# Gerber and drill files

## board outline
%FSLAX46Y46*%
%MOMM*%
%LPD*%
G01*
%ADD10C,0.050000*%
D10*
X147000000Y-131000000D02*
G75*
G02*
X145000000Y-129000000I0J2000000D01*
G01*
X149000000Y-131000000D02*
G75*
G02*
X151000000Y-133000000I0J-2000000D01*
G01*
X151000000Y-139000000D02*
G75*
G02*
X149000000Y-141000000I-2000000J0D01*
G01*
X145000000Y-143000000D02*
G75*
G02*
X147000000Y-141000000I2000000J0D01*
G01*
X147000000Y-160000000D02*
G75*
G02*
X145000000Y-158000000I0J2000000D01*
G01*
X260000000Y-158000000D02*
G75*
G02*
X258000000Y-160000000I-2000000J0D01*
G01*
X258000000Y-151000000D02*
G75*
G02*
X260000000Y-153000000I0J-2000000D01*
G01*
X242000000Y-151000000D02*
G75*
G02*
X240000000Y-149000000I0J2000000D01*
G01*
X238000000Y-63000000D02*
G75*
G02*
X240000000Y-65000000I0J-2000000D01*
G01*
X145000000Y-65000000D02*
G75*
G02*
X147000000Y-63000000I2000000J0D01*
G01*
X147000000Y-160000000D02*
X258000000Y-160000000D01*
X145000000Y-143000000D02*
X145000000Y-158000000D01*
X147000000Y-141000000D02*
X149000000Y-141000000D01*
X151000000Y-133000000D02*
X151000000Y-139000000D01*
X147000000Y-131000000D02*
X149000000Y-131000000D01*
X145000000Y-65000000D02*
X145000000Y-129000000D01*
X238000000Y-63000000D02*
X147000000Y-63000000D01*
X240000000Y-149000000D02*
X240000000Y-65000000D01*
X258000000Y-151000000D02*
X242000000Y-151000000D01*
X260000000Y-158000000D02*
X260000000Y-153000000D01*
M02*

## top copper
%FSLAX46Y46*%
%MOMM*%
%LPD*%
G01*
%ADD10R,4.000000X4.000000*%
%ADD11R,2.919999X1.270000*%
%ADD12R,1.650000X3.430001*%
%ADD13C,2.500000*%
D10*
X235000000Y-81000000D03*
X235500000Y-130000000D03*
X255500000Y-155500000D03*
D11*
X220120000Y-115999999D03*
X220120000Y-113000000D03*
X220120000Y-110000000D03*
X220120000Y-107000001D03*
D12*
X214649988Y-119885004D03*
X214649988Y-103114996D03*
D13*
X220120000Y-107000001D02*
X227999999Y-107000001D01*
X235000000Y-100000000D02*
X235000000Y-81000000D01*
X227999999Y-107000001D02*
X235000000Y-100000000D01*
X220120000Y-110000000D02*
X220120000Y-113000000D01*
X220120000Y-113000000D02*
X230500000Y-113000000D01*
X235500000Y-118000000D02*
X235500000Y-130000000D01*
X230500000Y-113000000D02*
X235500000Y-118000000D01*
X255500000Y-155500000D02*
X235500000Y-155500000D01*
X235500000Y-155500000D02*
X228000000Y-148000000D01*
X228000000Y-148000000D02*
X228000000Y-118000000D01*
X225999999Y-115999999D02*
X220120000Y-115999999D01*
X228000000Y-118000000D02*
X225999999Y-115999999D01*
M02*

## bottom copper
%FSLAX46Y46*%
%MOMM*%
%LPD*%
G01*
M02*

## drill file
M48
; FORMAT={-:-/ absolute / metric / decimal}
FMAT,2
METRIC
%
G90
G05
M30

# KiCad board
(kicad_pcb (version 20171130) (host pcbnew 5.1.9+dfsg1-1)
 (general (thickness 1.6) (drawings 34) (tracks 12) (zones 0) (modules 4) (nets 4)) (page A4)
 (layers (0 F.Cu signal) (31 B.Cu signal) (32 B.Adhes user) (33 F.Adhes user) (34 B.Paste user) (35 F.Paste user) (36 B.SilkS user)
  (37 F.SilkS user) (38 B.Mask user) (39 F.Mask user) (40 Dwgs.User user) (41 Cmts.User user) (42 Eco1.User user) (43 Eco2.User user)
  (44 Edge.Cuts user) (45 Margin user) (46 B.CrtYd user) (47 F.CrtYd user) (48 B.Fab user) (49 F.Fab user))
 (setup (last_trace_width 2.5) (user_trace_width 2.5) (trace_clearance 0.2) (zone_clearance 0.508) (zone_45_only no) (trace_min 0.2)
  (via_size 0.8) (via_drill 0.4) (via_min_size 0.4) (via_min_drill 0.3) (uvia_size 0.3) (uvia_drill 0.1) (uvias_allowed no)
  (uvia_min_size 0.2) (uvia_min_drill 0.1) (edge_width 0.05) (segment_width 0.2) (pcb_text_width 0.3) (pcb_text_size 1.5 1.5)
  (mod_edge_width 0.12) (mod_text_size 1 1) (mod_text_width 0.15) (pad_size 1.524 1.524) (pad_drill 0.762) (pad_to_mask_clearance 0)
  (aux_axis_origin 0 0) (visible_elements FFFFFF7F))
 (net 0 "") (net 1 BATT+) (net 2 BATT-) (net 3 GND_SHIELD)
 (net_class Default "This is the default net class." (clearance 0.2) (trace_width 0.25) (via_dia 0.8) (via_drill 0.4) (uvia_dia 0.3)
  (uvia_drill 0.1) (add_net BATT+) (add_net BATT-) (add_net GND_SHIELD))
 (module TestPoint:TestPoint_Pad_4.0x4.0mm (layer F.Cu) (at 235 81)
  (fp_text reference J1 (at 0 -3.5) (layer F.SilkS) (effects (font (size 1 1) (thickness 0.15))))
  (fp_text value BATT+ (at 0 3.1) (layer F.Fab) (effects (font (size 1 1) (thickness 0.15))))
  (pad 1 smd rect (at 0 0) (size 4 4) (layers F.Cu F.Mask) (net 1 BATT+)))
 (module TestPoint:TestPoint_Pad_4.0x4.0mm (layer F.Cu) (at 235.5 130)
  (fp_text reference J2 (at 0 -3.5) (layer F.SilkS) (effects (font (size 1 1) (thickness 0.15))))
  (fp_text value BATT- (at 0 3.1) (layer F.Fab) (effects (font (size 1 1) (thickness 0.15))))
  (pad 1 smd rect (at 0 0) (size 4 4) (layers F.Cu F.Mask) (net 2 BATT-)))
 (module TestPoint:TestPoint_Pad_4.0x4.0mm (layer F.Cu) (at 255.5 155.5)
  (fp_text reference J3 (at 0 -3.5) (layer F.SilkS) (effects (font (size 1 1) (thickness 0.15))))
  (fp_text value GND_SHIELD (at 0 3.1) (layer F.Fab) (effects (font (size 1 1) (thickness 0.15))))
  (pad 1 smd rect (at 0 0) (size 4 4) (layers F.Cu F.Mask) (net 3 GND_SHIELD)))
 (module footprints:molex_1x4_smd (layer F.Cu) (at 215 111.5 270)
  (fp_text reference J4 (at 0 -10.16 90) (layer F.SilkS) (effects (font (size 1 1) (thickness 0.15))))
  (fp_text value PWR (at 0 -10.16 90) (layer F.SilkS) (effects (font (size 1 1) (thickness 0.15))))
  (pad 1 smd rect (at 4.499999 -5.12 270) (size 1.27 2.919999) (layers F.Cu F.Paste F.Mask) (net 3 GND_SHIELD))
  (pad 2 smd rect (at 1.5 -5.12 270) (size 1.27 2.919999) (layers F.Cu F.Paste F.Mask) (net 2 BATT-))
  (pad 3 smd rect (at -1.5 -5.12 270) (size 1.27 2.919999) (layers F.Cu F.Paste F.Mask) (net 2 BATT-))
  (pad 4 smd rect (at -4.499999 -5.12 270) (size 1.27 2.919999) (layers F.Cu F.Paste F.Mask) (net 1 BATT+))
  (pad P1 smd rect (at 8.385004 0.350012 270) (size 3.430001 1.65) (layers F.Cu F.Paste F.Mask))
  (pad P2 smd rect (at -8.385004 0.350012 270) (size 3.430001 1.65) (layers F.Cu F.Paste F.Mask)))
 (gr_arc (start 147 129) (end 145 129) (angle -90) (layer Edge.Cuts) (width 0.05))
 (gr_arc (start 149 133) (end 151 133) (angle -90) (layer Edge.Cuts) (width 0.05))
 (gr_arc (start 149 139) (end 149 141) (angle -90) (layer Edge.Cuts) (width 0.05))
 (gr_arc (start 147 143) (end 147 141) (angle -90) (layer Edge.Cuts) (width 0.05))
 (gr_arc (start 147 158) (end 145 158) (angle -90) (layer Edge.Cuts) (width 0.05))
 (gr_arc (start 258 158) (end 258 160) (angle -90) (layer Edge.Cuts) (width 0.05))
 (gr_arc (start 258 153) (end 260 153) (angle -90) (layer Edge.Cuts) (width 0.05))
 (gr_arc (start 242 149) (end 240 149) (angle -90) (layer Edge.Cuts) (width 0.05))
 (gr_arc (start 238 65) (end 240 65) (angle -90) (layer Edge.Cuts) (width 0.05))
 (gr_arc (start 147 65) (end 147 63) (angle -90) (layer Edge.Cuts) (width 0.05))
 (gr_line (start 147 160) (end 258 160) (layer Edge.Cuts) (width 0.05))
 (gr_line (start 145 143) (end 145 158) (layer Edge.Cuts) (width 0.05))
 (gr_line (start 147 141) (end 149 141) (layer Edge.Cuts) (width 0.05))
 (gr_line (start 151 133) (end 151 139) (layer Edge.Cuts) (width 0.05))
 (gr_line (start 147 131) (end 149 131) (layer Edge.Cuts) (width 0.05))
 (gr_line (start 145 65) (end 145 129) (layer Edge.Cuts) (width 0.05))
 (gr_line (start 238 63) (end 147 63) (layer Edge.Cuts) (width 0.05))
 (gr_line (start 240 149) (end 240 65) (layer Edge.Cuts) (width 0.05))
 (gr_line (start 258 151) (end 242 151) (layer Edge.Cuts) (width 0.05))
 (gr_line (start 260 158) (end 260 153) (layer Edge.Cuts) (width 0.05))
 (segment (start 220.12 107.000001) (end 227.999999 107.000001) (width 2.5) (layer F.Cu) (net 1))
 (segment (start 235 100) (end 235 81) (width 2.5) (layer F.Cu) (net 1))
 (segment (start 227.999999 107.000001) (end 235 100) (width 2.5) (layer F.Cu) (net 1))
 (segment (start 220.12 110) (end 220.12 113) (width 2.5) (layer F.Cu) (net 2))
 (segment (start 220.12 113) (end 230.5 113) (width 2.5) (layer F.Cu) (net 2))
 (segment (start 235.5 118) (end 235.5 130) (width 2.5) (layer F.Cu) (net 2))
 (segment (start 230.5 113) (end 235.5 118) (width 2.5) (layer F.Cu) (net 2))
 (segment (start 255.5 155.5) (end 235.5 155.5) (width 2.5) (layer F.Cu) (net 3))
 (segment (start 235.5 155.5) (end 228 148) (width 2.5) (layer F.Cu) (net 3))
 (segment (start 228 148) (end 228 118) (width 2.5) (layer F.Cu) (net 3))
 (segment (start 225.999999 115.999999) (end 220.12 115.999999) (width 2.5) (layer F.Cu) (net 3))
 (segment (start 228 118) (end 225.999999 115.999999) (width 2.5) (layer F.Cu) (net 3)))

